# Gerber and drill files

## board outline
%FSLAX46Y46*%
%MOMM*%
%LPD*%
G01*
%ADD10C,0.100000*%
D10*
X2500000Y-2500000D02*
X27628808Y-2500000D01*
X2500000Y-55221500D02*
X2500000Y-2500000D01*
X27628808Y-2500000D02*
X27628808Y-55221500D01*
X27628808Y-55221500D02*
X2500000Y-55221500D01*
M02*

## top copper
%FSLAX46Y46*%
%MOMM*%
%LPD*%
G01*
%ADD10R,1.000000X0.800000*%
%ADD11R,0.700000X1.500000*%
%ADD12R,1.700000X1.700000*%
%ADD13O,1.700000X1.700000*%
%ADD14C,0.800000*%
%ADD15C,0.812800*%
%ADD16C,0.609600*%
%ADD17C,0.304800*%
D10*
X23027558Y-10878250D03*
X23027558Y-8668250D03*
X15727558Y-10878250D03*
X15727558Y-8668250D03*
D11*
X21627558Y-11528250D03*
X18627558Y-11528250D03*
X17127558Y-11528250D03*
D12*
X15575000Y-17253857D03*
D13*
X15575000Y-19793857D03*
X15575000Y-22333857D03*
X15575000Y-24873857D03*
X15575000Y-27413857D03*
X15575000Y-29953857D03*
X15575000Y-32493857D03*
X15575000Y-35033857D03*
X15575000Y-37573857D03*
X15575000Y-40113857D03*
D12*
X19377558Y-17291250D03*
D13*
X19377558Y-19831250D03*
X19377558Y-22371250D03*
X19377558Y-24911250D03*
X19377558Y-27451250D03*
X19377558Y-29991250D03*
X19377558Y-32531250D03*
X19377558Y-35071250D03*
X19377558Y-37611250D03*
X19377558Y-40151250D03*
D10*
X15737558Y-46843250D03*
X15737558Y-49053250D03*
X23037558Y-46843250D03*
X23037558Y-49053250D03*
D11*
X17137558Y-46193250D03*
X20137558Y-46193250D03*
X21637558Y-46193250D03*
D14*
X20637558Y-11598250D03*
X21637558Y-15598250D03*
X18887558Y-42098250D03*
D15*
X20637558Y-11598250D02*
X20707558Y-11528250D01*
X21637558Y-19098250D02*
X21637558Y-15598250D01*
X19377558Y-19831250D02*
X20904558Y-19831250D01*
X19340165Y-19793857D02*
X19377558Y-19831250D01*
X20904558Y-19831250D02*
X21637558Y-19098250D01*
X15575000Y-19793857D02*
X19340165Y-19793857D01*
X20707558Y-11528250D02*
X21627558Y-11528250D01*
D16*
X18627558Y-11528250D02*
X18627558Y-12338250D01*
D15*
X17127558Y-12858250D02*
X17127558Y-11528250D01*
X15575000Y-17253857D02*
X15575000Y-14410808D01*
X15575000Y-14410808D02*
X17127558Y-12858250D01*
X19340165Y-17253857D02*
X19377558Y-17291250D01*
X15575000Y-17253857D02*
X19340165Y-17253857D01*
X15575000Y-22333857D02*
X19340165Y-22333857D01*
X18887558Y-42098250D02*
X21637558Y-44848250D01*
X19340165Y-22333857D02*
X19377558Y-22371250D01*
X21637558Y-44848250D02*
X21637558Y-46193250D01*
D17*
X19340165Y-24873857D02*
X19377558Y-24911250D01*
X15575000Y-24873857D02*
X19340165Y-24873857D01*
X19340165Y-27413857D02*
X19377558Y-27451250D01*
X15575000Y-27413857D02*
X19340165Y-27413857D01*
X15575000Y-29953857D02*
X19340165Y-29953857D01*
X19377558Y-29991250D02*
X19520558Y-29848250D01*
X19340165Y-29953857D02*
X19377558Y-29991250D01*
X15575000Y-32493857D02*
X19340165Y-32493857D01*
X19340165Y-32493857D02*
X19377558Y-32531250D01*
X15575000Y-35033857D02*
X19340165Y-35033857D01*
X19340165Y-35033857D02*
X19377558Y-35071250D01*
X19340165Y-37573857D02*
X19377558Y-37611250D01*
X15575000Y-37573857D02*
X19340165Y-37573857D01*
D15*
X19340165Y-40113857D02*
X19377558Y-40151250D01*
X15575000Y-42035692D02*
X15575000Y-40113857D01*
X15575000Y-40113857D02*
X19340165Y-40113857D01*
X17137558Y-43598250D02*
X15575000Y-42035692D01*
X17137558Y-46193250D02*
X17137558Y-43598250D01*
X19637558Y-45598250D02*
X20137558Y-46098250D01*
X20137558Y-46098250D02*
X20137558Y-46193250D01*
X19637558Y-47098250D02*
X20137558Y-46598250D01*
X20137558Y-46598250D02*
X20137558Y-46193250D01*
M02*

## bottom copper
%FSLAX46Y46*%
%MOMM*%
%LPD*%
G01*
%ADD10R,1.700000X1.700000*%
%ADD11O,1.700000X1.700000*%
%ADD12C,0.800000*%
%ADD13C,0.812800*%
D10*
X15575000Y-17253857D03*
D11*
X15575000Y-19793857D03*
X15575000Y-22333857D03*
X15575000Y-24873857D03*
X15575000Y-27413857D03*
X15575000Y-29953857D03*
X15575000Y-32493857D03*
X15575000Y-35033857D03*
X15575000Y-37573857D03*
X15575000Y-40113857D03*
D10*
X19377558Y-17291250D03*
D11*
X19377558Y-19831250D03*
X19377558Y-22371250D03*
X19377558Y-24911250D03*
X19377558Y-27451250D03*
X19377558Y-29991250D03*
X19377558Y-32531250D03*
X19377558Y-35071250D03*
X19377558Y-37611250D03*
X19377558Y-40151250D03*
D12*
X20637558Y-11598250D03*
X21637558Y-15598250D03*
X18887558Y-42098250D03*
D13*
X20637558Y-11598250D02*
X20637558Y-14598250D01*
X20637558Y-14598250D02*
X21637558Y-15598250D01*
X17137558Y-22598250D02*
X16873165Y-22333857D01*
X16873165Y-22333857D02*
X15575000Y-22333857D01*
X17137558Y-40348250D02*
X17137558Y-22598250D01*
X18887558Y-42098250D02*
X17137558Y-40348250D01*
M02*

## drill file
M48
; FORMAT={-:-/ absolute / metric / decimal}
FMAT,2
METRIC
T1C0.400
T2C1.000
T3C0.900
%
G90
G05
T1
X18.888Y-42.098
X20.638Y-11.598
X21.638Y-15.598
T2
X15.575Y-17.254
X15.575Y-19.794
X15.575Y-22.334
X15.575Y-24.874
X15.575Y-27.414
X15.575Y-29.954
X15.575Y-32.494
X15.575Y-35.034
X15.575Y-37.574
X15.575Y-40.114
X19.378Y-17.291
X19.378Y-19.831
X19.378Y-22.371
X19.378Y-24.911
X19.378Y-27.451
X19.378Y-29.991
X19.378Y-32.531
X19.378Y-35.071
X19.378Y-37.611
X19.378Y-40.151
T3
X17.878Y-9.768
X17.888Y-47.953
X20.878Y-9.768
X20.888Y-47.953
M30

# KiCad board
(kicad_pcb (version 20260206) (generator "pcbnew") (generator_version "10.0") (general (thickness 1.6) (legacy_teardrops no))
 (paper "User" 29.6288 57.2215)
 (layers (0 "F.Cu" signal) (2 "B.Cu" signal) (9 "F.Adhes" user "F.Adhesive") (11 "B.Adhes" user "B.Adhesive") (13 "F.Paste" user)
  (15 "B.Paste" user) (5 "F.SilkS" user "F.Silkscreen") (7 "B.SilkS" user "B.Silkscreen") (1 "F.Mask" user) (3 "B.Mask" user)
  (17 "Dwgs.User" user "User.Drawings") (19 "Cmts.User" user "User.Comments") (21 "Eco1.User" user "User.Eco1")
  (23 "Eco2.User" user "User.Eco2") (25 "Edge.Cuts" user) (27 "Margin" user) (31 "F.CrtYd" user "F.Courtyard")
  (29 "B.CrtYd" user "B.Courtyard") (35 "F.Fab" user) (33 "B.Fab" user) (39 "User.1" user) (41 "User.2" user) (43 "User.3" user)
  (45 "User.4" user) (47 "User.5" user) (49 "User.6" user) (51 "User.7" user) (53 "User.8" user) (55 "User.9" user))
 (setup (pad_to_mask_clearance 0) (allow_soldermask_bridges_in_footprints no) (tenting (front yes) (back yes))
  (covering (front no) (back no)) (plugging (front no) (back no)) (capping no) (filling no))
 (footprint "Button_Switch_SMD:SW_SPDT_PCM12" (layer "F.Cu") (at 19.377558 10.09825 180)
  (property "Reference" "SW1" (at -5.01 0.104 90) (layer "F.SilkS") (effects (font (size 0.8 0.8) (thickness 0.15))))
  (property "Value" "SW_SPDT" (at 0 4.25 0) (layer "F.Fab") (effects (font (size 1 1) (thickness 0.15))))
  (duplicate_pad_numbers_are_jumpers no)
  (pad "" smd rect (at -3.65 -0.78 180) (size 1 0.8) (layers "F.Cu" "F.Mask" "F.Paste"))
  (pad "" smd rect (at -3.65 1.43 180) (size 1 0.8) (layers "F.Cu" "F.Mask" "F.Paste"))
  (pad "" np_thru_hole circle (at -1.5 0.33 180) (size 0.9 0.9) (drill 0.9) (layers "*.Cu" "*.Mask"))
  (pad "" np_thru_hole circle (at 1.5 0.33 180) (size 0.9 0.9) (drill 0.9) (layers "*.Cu" "*.Mask"))
  (pad "" smd rect (at 3.65 -0.78 180) (size 1 0.8) (layers "F.Cu" "F.Mask" "F.Paste"))
  (pad "" smd rect (at 3.65 1.43 180) (size 1 0.8) (layers "F.Cu" "F.Mask" "F.Paste"))
  (pad "1" smd rect (at -2.25 -1.43 180) (size 0.7 1.5) (layers "F.Cu" "F.Mask" "F.Paste") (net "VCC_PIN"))
  (pad "2" smd rect (at 0.75 -1.43 180) (size 0.7 1.5) (layers "F.Cu" "F.Mask" "F.Paste") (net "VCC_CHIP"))
  (pad "3" smd rect (at 2.25 -1.43 180) (size 0.7 1.5) (layers "F.Cu" "F.Mask" "F.Paste") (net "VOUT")))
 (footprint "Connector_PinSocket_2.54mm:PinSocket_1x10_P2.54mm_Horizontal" (layer "F.Cu") (at 15.575 17.253857)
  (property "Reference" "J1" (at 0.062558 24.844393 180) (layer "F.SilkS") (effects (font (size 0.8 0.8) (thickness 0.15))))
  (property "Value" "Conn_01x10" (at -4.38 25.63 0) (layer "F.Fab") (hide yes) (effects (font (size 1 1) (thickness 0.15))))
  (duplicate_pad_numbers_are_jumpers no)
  (pad "1" thru_hole rect (at 0 0) (size 1.7 1.7) (drill 1) (layers "*.Cu" "*.Mask") (remove_unused_layers no) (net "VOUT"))
  (pad "2" thru_hole oval (at 0 2.54) (size 1.7 1.7) (drill 1) (layers "*.Cu" "*.Mask") (remove_unused_layers no) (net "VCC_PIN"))
  (pad "3" thru_hole oval (at 0 5.08) (size 1.7 1.7) (drill 1) (layers "*.Cu" "*.Mask") (remove_unused_layers no) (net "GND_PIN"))
  (pad "4" thru_hole oval (at 0 7.62) (size 1.7 1.7) (drill 1) (layers "*.Cu" "*.Mask") (remove_unused_layers no) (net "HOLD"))
  (pad "5" thru_hole oval (at 0 10.16) (size 1.7 1.7) (drill 1) (layers "*.Cu" "*.Mask") (remove_unused_layers no) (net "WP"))
  (pad "6" thru_hole oval (at 0 12.7) (size 1.7 1.7) (drill 1) (layers "*.Cu" "*.Mask") (remove_unused_layers no) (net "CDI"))
  (pad "7" thru_hole oval (at 0 15.24) (size 1.7 1.7) (drill 1) (layers "*.Cu" "*.Mask") (remove_unused_layers no) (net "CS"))
  (pad "8" thru_hole oval (at 0 17.78) (size 1.7 1.7) (drill 1) (layers "*.Cu" "*.Mask") (remove_unused_layers no) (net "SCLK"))
  (pad "9" thru_hole oval (at 0 20.32) (size 1.7 1.7) (drill 1) (layers "*.Cu" "*.Mask") (remove_unused_layers no) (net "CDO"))
  (pad "10" thru_hole oval (at 0 22.86) (size 1.7 1.7) (drill 1) (layers "*.Cu" "*.Mask") (remove_unused_layers no) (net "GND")))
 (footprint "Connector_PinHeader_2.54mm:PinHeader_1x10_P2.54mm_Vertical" (layer "F.Cu") (at 19.377558 17.29125)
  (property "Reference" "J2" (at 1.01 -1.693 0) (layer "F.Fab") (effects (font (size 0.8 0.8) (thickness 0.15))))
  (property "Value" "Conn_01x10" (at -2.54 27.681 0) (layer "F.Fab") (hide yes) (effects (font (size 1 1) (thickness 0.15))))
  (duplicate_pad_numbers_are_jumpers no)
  (pad "1" thru_hole rect (at 0 0) (size 1.7 1.7) (drill 1) (layers "*.Cu" "*.Mask") (remove_unused_layers no) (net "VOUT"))
  (pad "2" thru_hole oval (at 0 2.54) (size 1.7 1.7) (drill 1) (layers "*.Cu" "*.Mask") (remove_unused_layers no) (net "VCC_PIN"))
  (pad "3" thru_hole oval (at 0 5.08) (size 1.7 1.7) (drill 1) (layers "*.Cu" "*.Mask") (remove_unused_layers no) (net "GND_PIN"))
  (pad "4" thru_hole oval (at 0 7.62) (size 1.7 1.7) (drill 1) (layers "*.Cu" "*.Mask") (remove_unused_layers no) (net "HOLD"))
  (pad "5" thru_hole oval (at 0 10.16) (size 1.7 1.7) (drill 1) (layers "*.Cu" "*.Mask") (remove_unused_layers no) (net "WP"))
  (pad "6" thru_hole oval (at 0 12.7) (size 1.7 1.7) (drill 1) (layers "*.Cu" "*.Mask") (remove_unused_layers no) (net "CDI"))
  (pad "7" thru_hole oval (at 0 15.24) (size 1.7 1.7) (drill 1) (layers "*.Cu" "*.Mask") (remove_unused_layers no) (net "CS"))
  (pad "8" thru_hole oval (at 0 17.78) (size 1.7 1.7) (drill 1) (layers "*.Cu" "*.Mask") (remove_unused_layers no) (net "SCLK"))
  (pad "9" thru_hole oval (at 0 20.32) (size 1.7 1.7) (drill 1) (layers "*.Cu" "*.Mask") (remove_unused_layers no) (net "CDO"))
  (pad "10" thru_hole oval (at 0 22.86) (size 1.7 1.7) (drill 1) (layers "*.Cu" "*.Mask") (remove_unused_layers no) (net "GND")))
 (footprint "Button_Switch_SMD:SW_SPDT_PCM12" (layer "F.Cu") (at 19.387558 47.62325)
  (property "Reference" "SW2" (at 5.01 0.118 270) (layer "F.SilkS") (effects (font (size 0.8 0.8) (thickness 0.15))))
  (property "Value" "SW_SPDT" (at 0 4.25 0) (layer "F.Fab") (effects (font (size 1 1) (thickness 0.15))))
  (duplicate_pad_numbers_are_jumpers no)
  (pad "" smd rect (at -3.65 -0.78) (size 1 0.8) (layers "F.Cu" "F.Mask" "F.Paste"))
  (pad "" smd rect (at -3.65 1.43) (size 1 0.8) (layers "F.Cu" "F.Mask" "F.Paste"))
  (pad "" np_thru_hole circle (at -1.5 0.33) (size 0.9 0.9) (drill 0.9) (layers "*.Cu" "*.Mask"))
  (pad "" np_thru_hole circle (at 1.5 0.33) (size 0.9 0.9) (drill 0.9) (layers "*.Cu" "*.Mask"))
  (pad "" smd rect (at 3.65 -0.78) (size 1 0.8) (layers "F.Cu" "F.Mask" "F.Paste"))
  (pad "" smd rect (at 3.65 1.43) (size 1 0.8) (layers "F.Cu" "F.Mask" "F.Paste"))
  (pad "1" smd rect (at -2.25 -1.43) (size 0.7 1.5) (layers "F.Cu" "F.Mask" "F.Paste") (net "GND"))
  (pad "2" smd rect (at 0.75 -1.43) (size 0.7 1.5) (layers "F.Cu" "F.Mask" "F.Paste") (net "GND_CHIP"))
  (pad "3" smd rect (at 2.25 -1.43) (size 0.7 1.5) (layers "F.Cu" "F.Mask" "F.Paste") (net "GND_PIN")))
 (gr_line (start 2.5 2.5) (end 27.628808 2.5) (stroke (width 0.1) (type default)) (layer "Edge.Cuts"))
 (gr_line (start 2.5 55.2215) (end 2.5 2.5) (stroke (width 0.1) (type default)) (layer "Edge.Cuts"))
 (gr_line (start 27.628808 2.5) (end 27.628808 55.2215) (stroke (width 0.1) (type default)) (layer "Edge.Cuts"))
 (gr_line (start 27.628808 55.2215) (end 2.5 55.2215) (stroke (width 0.1) (type default)) (layer "Edge.Cuts"))
 (segment (start 20.637558 11.59825) (end 20.707558 11.52825) (width 0.8128) (layer "F.Cu") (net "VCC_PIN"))
 (segment (start 21.637558 19.09825) (end 21.637558 15.59825) (width 0.8128) (layer "F.Cu") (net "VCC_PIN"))
 (segment (start 19.377558 19.83125) (end 20.904558 19.83125) (width 0.8128) (layer "F.Cu") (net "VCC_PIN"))
 (segment (start 19.340165 19.793857) (end 19.377558 19.83125) (width 0.8128) (layer "F.Cu") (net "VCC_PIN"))
 (segment (start 20.904558 19.83125) (end 21.637558 19.09825) (width 0.8128) (layer "F.Cu") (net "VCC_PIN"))
 (segment (start 15.575 19.793857) (end 19.340165 19.793857) (width 0.8128) (layer "F.Cu") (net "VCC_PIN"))
 (segment (start 20.707558 11.52825) (end 21.627558 11.52825) (width 0.8128) (layer "F.Cu") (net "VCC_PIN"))
 (via (at 20.637558 11.59825) (size 0.8) (drill 0.4) (layers "F.Cu" "B.Cu") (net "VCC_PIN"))
 (via (at 21.637558 15.59825) (size 0.8) (drill 0.4) (layers "F.Cu" "B.Cu") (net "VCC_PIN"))
 (segment (start 20.637558 11.59825) (end 20.637558 14.59825) (width 0.8128) (layer "B.Cu") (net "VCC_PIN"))
 (segment (start 20.637558 14.59825) (end 21.637558 15.59825) (width 0.8128) (layer "B.Cu") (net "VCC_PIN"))
 (segment (start 18.627558 11.52825) (end 18.627558 12.33825) (width 0.6096) (layer "F.Cu") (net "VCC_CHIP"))
 (segment (start 17.127558 12.85825) (end 17.127558 11.52825) (width 0.8128) (layer "F.Cu") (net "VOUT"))
 (segment (start 15.575 17.253857) (end 15.575 14.410808) (width 0.8128) (layer "F.Cu") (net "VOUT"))
 (segment (start 15.575 14.410808) (end 17.127558 12.85825) (width 0.8128) (layer "F.Cu") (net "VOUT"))
 (segment (start 19.340165 17.253857) (end 19.377558 17.29125) (width 0.8128) (layer "F.Cu") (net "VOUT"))
 (segment (start 15.575 17.253857) (end 19.340165 17.253857) (width 0.8128) (layer "F.Cu") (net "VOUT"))
 (segment (start 15.575 22.333857) (end 19.340165 22.333857) (width 0.8128) (layer "F.Cu") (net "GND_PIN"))
 (segment (start 18.887558 42.09825) (end 21.637558 44.84825) (width 0.8128) (layer "F.Cu") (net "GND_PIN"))
 (segment (start 19.340165 22.333857) (end 19.377558 22.37125) (width 0.8128) (layer "F.Cu") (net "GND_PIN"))
 (segment (start 21.637558 44.84825) (end 21.637558 46.19325) (width 0.8128) (layer "F.Cu") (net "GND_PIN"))
 (via (at 18.887558 42.09825) (size 0.8) (drill 0.4) (layers "F.Cu" "B.Cu") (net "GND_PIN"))
 (segment (start 17.137558 22.59825) (end 16.873165 22.333857) (width 0.8128) (layer "B.Cu") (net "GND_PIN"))
 (segment (start 16.873165 22.333857) (end 15.575 22.333857) (width 0.8128) (layer "B.Cu") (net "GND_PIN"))
 (segment (start 17.137558 40.34825) (end 17.137558 22.59825) (width 0.8128) (layer "B.Cu") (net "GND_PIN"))
 (segment (start 18.887558 42.09825) (end 17.137558 40.34825) (width 0.8128) (layer "B.Cu") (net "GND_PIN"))
 (segment (start 19.340165 24.873857) (end 19.377558 24.91125) (width 0.3048) (layer "F.Cu") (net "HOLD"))
 (segment (start 15.575 24.873857) (end 19.340165 24.873857) (width 0.3048) (layer "F.Cu") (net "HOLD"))
 (segment (start 19.340165 27.413857) (end 19.377558 27.45125) (width 0.3048) (layer "F.Cu") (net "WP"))
 (segment (start 15.575 27.413857) (end 19.340165 27.413857) (width 0.3048) (layer "F.Cu") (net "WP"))
 (segment (start 15.575 29.953857) (end 19.340165 29.953857) (width 0.3048) (layer "F.Cu") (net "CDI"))
 (segment (start 19.377558 29.99125) (end 19.520558 29.84825) (width 0.3048) (layer "F.Cu") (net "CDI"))
 (segment (start 19.340165 29.953857) (end 19.377558 29.99125) (width 0.3048) (layer "F.Cu") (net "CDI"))
 (segment (start 15.575 32.493857) (end 19.340165 32.493857) (width 0.3048) (layer "F.Cu") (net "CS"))
 (segment (start 19.340165 32.493857) (end 19.377558 32.53125) (width 0.3048) (layer "F.Cu") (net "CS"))
 (segment (start 15.575 35.033857) (end 19.340165 35.033857) (width 0.3048) (layer "F.Cu") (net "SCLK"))
 (segment (start 19.340165 35.033857) (end 19.377558 35.07125) (width 0.3048) (layer "F.Cu") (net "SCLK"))
 (segment (start 19.340165 37.573857) (end 19.377558 37.61125) (width 0.3048) (layer "F.Cu") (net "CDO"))
 (segment (start 15.575 37.573857) (end 19.340165 37.573857) (width 0.3048) (layer "F.Cu") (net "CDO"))
 (segment (start 19.340165 40.113857) (end 19.377558 40.15125) (width 0.8128) (layer "F.Cu") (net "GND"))
 (segment (start 15.575 42.035692) (end 15.575 40.113857) (width 0.8128) (layer "F.Cu") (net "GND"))
 (segment (start 15.575 40.113857) (end 19.340165 40.113857) (width 0.8128) (layer "F.Cu") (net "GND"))
 (segment (start 17.137558 43.59825) (end 15.575 42.035692) (width 0.8128) (layer "F.Cu") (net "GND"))
 (segment (start 17.137558 46.19325) (end 17.137558 43.59825) (width 0.8128) (layer "F.Cu") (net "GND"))
 (segment (start 19.637558 45.59825) (end 20.137558 46.09825) (width 0.8128) (layer "F.Cu") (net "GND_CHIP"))
 (segment (start 20.137558 46.09825) (end 20.137558 46.19325) (width 0.8128) (layer "F.Cu") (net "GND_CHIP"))
 (segment (start 19.637558 47.09825) (end 20.137558 46.59825) (width 0.8128) (layer "F.Cu") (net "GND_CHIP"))
 (segment (start 20.137558 46.59825) (end 20.137558 46.19325) (width 0.8128) (layer "F.Cu") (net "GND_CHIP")))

